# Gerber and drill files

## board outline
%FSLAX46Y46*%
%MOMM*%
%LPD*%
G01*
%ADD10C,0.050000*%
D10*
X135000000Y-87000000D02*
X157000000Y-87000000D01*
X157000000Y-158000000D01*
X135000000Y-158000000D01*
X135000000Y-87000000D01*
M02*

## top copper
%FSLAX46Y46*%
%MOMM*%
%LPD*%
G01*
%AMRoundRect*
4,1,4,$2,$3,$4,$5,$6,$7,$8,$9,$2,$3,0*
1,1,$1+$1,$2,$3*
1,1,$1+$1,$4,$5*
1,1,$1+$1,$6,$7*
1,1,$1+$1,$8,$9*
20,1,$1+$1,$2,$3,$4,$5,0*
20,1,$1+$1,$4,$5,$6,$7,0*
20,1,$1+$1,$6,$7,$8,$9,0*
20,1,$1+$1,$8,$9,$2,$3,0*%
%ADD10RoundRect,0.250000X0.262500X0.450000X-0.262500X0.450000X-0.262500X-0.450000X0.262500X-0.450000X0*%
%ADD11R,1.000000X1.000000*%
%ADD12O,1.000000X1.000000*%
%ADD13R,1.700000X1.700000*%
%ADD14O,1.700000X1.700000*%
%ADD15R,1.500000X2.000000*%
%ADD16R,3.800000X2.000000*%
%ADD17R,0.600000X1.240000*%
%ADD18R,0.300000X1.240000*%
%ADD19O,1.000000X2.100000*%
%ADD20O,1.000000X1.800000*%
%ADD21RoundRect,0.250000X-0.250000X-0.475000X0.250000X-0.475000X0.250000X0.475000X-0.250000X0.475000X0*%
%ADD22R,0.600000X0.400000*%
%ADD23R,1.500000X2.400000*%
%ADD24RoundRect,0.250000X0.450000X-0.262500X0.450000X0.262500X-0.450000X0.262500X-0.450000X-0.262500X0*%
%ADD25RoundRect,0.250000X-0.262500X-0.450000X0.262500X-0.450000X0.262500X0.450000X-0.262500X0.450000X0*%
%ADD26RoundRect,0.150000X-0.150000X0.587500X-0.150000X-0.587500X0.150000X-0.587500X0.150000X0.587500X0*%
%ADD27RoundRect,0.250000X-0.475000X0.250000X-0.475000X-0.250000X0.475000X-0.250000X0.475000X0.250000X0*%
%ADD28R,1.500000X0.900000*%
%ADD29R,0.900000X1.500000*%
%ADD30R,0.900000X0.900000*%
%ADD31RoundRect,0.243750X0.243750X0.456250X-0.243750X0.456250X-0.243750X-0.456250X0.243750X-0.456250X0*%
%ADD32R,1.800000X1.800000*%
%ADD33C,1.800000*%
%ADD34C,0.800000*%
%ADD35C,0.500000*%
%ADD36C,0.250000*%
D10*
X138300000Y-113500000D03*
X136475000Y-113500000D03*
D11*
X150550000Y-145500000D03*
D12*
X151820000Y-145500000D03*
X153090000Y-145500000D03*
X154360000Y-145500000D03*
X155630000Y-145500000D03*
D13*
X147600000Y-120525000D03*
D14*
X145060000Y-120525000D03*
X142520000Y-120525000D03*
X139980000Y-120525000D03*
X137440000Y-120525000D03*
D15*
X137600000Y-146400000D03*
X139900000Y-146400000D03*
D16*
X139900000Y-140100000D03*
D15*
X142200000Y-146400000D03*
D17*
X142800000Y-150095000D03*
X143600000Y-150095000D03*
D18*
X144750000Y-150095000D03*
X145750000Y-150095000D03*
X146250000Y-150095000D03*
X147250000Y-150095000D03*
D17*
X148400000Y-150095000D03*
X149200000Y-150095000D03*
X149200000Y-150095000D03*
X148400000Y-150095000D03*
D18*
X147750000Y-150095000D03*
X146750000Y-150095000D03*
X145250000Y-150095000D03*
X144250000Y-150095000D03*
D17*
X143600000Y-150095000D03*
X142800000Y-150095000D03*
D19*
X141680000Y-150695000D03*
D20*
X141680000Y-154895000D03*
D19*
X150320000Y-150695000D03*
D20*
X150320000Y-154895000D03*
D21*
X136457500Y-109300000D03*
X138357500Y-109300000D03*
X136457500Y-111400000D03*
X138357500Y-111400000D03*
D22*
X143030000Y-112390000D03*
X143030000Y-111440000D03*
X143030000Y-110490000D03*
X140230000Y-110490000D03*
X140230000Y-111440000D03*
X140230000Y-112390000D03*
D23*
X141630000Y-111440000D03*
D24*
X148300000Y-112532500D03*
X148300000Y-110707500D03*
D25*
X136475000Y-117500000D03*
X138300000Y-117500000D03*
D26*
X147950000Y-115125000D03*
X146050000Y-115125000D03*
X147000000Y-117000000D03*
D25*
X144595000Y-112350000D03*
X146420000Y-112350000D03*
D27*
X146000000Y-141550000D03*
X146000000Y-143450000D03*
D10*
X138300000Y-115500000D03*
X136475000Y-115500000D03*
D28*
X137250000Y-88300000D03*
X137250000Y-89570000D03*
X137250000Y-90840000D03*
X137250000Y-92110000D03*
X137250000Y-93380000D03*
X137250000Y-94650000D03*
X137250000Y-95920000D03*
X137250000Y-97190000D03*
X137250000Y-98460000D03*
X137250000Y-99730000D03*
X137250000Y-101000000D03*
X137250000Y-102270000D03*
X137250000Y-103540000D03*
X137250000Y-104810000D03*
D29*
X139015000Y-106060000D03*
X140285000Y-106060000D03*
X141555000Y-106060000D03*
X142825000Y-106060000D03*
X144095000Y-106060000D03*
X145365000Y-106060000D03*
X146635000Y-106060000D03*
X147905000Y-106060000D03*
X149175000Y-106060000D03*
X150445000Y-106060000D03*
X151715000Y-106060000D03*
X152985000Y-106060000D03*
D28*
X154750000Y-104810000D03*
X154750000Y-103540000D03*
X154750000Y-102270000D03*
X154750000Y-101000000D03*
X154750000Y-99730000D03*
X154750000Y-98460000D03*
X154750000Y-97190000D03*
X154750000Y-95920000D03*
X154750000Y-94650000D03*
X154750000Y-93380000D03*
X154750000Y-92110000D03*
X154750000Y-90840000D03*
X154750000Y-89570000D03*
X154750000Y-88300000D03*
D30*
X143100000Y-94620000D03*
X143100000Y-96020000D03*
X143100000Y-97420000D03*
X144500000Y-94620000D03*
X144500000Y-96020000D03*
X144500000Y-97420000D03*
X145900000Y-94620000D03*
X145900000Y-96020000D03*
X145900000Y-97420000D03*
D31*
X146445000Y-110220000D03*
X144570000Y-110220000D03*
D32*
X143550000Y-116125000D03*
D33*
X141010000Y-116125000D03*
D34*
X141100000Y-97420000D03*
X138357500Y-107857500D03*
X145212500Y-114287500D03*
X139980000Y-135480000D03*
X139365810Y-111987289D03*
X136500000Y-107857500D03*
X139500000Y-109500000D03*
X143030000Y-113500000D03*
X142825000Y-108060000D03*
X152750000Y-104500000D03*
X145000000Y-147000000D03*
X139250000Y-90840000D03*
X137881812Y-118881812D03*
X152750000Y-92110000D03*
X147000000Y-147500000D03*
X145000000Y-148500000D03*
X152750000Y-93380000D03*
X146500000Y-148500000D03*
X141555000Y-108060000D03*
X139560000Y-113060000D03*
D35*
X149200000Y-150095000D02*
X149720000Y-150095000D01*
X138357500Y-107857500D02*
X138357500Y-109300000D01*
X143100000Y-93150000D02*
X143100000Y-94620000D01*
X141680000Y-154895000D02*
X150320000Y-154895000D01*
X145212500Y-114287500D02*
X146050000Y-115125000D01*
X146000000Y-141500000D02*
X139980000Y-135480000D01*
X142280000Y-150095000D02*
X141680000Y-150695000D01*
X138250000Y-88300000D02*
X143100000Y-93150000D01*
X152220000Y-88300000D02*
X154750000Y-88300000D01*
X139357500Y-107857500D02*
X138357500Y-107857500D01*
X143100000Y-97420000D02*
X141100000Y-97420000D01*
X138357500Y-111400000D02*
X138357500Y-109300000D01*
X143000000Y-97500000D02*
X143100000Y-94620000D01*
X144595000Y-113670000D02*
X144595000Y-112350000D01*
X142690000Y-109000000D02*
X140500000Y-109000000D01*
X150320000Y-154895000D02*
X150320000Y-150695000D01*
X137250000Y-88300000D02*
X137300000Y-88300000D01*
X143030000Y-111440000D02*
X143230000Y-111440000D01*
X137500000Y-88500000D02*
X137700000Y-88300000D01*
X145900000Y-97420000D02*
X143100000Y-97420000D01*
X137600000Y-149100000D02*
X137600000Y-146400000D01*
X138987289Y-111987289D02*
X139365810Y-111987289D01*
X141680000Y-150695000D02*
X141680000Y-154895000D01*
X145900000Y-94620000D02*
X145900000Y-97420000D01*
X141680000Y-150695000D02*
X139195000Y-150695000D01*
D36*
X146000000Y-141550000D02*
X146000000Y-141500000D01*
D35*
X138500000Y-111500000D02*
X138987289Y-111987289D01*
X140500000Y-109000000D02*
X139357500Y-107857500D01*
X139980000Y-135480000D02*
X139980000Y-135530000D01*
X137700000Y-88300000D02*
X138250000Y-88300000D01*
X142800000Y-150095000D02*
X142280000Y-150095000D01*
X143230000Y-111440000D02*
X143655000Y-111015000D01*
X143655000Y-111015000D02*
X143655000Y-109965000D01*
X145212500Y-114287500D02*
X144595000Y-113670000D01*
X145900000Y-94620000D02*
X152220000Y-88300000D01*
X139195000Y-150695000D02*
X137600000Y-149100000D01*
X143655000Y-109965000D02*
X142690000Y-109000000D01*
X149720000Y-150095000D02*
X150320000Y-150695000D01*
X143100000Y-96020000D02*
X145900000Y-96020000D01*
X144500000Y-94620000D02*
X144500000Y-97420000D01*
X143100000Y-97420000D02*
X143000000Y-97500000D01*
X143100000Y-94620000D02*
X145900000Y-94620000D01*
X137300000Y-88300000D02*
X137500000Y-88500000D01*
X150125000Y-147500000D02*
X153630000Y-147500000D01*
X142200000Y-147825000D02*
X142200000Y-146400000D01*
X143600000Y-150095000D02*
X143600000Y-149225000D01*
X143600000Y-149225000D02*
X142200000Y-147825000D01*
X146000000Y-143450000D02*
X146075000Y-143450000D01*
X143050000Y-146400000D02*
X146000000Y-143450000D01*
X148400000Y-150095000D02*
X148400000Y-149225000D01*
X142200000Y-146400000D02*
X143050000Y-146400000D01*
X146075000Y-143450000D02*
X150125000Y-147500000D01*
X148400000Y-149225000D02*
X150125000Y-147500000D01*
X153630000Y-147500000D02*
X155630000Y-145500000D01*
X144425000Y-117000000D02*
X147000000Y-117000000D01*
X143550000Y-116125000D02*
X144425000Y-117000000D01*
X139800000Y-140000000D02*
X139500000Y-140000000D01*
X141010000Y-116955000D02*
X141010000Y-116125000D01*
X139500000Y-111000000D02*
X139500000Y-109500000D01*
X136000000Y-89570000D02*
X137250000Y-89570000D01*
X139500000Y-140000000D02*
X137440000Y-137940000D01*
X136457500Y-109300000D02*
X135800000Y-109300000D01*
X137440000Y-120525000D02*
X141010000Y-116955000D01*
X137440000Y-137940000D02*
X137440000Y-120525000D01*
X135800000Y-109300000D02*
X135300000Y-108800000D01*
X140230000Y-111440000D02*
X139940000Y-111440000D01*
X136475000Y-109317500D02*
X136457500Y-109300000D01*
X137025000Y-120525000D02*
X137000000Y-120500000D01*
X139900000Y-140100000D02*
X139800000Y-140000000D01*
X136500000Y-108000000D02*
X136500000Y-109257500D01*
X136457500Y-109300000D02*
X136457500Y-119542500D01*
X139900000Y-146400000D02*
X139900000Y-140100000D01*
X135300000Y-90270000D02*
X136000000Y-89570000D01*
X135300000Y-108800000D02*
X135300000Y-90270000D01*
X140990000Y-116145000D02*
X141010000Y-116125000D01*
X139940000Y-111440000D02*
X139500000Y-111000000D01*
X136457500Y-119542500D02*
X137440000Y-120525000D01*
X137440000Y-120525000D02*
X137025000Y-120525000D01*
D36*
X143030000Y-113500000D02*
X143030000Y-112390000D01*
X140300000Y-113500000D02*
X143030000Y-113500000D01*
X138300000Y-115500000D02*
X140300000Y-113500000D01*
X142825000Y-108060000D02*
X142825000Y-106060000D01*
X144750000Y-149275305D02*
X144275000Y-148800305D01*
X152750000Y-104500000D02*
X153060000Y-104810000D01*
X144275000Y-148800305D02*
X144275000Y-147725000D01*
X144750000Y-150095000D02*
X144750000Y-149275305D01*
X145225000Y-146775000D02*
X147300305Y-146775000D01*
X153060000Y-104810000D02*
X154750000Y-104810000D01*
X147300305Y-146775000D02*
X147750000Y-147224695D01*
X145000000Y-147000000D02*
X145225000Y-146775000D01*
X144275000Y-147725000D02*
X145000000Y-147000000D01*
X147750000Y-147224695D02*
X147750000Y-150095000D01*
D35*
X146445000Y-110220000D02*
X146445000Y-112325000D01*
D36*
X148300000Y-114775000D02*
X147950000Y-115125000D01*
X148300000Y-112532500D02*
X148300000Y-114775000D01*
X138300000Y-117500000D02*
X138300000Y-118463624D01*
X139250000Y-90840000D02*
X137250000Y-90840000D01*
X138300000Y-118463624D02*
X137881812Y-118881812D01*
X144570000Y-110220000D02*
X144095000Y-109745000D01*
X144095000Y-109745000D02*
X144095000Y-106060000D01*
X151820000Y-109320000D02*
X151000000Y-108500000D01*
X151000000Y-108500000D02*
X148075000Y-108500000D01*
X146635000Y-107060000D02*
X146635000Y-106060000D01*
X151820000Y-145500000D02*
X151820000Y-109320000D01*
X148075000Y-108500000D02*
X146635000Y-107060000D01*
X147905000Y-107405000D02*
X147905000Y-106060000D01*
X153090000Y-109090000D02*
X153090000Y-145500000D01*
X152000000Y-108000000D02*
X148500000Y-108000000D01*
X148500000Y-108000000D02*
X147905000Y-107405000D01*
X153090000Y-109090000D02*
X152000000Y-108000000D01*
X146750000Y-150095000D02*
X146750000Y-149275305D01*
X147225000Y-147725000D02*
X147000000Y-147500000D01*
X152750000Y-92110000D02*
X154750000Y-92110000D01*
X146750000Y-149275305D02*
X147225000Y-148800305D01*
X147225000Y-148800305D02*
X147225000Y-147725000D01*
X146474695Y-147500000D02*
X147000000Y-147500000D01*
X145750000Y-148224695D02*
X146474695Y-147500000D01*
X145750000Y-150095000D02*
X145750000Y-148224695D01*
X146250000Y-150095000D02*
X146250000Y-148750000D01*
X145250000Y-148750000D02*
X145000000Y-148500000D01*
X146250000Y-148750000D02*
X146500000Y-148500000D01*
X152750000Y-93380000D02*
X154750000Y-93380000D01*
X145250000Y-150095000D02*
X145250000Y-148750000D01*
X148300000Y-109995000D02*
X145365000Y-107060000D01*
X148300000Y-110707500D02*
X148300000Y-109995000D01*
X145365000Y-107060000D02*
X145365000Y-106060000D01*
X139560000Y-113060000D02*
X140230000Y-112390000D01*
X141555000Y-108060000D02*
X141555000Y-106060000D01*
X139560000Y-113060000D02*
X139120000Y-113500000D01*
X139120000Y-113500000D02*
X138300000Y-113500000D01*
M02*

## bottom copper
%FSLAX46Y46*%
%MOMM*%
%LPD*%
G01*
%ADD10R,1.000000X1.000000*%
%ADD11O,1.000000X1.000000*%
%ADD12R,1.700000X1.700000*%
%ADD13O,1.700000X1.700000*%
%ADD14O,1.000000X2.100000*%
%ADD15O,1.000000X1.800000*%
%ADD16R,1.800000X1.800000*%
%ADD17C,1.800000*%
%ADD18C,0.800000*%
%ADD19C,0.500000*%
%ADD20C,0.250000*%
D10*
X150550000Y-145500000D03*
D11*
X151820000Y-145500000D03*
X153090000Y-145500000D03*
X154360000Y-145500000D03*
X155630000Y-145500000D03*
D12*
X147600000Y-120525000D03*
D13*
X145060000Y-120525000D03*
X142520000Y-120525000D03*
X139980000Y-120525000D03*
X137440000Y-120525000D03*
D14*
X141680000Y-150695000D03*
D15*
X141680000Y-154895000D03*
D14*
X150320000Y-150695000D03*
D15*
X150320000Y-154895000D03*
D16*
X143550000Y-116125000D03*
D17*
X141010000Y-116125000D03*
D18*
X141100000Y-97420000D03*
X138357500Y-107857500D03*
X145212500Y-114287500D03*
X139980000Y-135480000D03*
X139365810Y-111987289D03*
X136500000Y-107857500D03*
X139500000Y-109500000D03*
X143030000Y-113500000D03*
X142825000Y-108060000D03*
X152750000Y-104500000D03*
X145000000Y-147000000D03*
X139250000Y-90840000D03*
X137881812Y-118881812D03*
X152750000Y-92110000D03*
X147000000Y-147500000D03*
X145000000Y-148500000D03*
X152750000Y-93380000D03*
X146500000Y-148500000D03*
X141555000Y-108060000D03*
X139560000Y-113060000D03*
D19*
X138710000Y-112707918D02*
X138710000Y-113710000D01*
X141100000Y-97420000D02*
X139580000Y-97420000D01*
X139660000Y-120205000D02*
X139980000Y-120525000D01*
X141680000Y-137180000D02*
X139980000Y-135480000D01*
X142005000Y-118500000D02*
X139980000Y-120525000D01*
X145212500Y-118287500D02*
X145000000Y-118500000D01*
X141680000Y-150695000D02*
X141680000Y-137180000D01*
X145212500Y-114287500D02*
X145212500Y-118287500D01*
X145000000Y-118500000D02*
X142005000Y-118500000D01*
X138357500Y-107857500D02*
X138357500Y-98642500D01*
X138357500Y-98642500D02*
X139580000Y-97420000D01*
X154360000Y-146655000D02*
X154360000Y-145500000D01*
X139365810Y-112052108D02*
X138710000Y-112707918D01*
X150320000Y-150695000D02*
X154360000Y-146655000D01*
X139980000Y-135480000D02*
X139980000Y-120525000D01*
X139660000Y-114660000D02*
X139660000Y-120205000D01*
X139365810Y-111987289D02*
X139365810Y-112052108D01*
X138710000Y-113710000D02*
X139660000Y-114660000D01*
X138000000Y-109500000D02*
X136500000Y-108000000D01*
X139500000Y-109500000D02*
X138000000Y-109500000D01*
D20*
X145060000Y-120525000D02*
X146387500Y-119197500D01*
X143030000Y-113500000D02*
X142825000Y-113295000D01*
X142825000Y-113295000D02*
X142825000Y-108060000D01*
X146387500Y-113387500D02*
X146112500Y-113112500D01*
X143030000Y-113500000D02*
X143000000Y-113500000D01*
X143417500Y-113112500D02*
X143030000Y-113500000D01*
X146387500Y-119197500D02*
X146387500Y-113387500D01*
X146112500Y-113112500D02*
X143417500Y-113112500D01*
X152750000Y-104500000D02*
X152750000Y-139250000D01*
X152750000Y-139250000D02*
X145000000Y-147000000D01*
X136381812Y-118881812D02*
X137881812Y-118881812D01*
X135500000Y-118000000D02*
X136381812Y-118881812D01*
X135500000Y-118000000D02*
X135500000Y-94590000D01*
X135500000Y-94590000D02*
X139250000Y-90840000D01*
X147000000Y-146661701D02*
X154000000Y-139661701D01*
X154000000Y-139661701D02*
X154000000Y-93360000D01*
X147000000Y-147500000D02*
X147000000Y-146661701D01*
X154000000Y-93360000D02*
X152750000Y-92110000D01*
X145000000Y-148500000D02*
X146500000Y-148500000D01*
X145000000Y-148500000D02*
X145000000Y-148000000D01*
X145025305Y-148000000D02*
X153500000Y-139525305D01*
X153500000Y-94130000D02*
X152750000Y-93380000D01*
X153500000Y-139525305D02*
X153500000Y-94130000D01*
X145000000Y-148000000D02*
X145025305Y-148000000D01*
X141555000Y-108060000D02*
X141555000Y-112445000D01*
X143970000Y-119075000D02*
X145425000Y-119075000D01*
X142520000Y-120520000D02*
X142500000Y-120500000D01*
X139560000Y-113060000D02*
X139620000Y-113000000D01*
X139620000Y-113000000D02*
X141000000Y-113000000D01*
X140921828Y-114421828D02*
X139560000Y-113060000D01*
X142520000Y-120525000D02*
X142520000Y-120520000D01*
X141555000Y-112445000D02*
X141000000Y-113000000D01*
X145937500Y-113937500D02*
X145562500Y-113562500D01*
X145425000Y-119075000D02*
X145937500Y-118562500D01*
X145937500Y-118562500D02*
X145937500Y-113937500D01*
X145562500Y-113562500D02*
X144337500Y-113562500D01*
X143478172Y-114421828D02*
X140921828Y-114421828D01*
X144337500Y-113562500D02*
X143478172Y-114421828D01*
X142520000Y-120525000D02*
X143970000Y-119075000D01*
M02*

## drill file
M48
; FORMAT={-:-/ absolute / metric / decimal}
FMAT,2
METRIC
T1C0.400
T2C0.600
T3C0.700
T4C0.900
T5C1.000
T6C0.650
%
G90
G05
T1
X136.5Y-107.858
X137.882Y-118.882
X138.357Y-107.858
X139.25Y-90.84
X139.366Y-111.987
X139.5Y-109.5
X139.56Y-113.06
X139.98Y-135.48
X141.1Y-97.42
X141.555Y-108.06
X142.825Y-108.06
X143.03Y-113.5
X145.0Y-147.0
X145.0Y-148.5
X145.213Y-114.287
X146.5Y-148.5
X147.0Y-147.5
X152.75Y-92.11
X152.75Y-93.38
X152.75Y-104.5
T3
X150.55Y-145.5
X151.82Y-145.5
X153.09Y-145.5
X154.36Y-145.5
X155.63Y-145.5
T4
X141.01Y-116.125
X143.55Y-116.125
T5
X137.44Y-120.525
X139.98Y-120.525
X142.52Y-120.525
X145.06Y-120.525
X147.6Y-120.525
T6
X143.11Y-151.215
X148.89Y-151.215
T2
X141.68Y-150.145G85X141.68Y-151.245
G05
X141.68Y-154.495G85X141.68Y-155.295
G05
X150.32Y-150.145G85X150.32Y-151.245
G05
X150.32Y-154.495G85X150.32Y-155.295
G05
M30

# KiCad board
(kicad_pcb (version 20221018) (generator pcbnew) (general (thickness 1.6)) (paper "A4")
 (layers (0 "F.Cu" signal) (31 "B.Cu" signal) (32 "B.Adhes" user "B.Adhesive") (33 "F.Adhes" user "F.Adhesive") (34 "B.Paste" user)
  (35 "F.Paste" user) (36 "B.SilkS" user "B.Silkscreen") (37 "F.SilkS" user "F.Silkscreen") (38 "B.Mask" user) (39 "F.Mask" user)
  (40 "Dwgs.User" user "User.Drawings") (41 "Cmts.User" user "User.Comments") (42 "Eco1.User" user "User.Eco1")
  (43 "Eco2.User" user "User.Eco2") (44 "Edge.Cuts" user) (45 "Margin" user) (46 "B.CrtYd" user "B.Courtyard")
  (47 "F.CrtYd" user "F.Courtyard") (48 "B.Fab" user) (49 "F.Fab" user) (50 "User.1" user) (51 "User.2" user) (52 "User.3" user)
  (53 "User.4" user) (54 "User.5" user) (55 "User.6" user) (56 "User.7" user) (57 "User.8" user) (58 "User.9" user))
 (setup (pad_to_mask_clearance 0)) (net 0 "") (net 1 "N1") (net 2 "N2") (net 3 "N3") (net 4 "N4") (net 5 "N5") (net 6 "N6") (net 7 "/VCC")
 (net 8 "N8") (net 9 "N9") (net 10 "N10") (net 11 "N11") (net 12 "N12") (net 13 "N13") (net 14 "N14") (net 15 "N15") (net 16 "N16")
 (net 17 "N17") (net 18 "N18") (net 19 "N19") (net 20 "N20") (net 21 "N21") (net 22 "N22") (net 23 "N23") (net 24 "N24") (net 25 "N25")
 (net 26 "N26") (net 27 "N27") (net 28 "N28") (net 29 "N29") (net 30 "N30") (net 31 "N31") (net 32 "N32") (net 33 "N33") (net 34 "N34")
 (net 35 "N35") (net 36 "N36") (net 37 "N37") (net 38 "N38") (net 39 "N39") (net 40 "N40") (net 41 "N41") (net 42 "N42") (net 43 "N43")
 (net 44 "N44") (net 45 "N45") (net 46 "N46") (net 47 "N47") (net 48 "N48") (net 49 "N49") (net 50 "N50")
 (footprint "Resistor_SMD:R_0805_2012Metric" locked (layer "F.Cu") (at 137.3875 113.5 180)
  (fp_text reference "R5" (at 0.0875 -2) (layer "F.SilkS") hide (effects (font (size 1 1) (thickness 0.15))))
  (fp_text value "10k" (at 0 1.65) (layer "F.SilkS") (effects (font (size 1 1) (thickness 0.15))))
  (pad "1" smd roundrect locked (at -0.9125 0 180) (size 1.025 1.4) (layers "F.Cu" "F.Paste" "F.Mask") (roundrect_rratio 0.243902439)
   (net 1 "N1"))
  (pad "2" smd roundrect locked (at 0.9125 0 180) (size 1.025 1.4) (layers "F.Cu" "F.Paste" "F.Mask") (roundrect_rratio 0.243902439)
   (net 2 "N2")))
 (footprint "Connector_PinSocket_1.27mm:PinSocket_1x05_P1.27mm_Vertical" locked (layer "F.Cu") (at 150.55 145.5 90)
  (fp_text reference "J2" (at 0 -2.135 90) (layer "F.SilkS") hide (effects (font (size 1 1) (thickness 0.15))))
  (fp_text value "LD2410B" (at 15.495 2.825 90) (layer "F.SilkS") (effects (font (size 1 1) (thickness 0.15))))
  (pad "1" thru_hole rect locked (at 0 0 90) (size 1 1) (drill 0.7) (layers "*.Cu" "*.Mask") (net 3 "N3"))
  (pad "2" thru_hole oval locked (at 0 1.27 90) (size 1 1) (drill 0.7) (layers "*.Cu" "*.Mask") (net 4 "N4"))
  (pad "3" thru_hole oval locked (at 0 2.54 90) (size 1 1) (drill 0.7) (layers "*.Cu" "*.Mask") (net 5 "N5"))
  (pad "4" thru_hole oval locked (at 0 3.81 90) (size 1 1) (drill 0.7) (layers "*.Cu" "*.Mask") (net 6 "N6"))
  (pad "5" thru_hole oval locked (at 0 5.08 90) (size 1 1) (drill 0.7) (layers "*.Cu" "*.Mask") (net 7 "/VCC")))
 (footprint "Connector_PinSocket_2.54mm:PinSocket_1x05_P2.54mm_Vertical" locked (layer "F.Cu") (at 147.6 120.525 -90)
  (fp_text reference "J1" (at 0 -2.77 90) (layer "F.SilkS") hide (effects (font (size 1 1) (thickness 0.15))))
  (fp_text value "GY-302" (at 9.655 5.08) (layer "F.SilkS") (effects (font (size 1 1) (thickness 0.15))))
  (pad "1" thru_hole rect locked (at 0 0 270) (size 1.7 1.7) (drill 1) (layers "*.Cu" "*.Mask") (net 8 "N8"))
  (pad "2" thru_hole oval locked (at 0 2.54 270) (size 1.7 1.7) (drill 1) (layers "*.Cu" "*.Mask") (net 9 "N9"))
  (pad "3" thru_hole oval locked (at 0 5.08 270) (size 1.7 1.7) (drill 1) (layers "*.Cu" "*.Mask") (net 1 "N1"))
  (pad "4" thru_hole oval locked (at 0 7.62 270) (size 1.7 1.7) (drill 1) (layers "*.Cu" "*.Mask") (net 6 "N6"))
  (pad "5" thru_hole oval locked (at 0 10.16 270) (size 1.7 1.7) (drill 1) (layers "*.Cu" "*.Mask") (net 2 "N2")))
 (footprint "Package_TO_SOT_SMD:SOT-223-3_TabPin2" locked (layer "F.Cu") (at 139.9 143.25 90)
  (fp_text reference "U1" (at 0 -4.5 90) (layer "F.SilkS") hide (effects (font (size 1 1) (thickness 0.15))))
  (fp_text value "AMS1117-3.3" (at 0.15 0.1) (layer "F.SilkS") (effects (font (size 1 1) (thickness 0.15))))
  (pad "1" smd rect locked (at -3.15 -2.3 90) (size 2 1.5) (layers "F.Cu" "F.Paste" "F.Mask") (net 6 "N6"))
  (pad "2" smd rect locked (at -3.15 0 90) (size 2 1.5) (layers "F.Cu" "F.Paste" "F.Mask") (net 2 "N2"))
  (pad "2" smd rect locked (at 3.15 0 90) (size 2 3.8) (layers "F.Cu" "F.Paste" "F.Mask") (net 2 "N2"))
  (pad "3" smd rect locked (at -3.15 2.3 90) (size 2 1.5) (layers "F.Cu" "F.Paste" "F.Mask") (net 7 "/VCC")))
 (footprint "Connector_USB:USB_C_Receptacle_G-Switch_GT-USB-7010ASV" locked (layer "F.Cu") (at 146 153.82)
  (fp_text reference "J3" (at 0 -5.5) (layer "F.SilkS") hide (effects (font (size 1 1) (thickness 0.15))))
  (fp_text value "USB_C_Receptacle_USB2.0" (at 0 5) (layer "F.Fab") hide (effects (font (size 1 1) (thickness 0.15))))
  (pad "" np_thru_hole circle locked (at -2.89 -2.605) (size 0.65 0.65) (drill 0.65) (layers "*.Cu" "*.Mask"))
  (pad "" np_thru_hole circle locked (at 2.89 -2.605) (size 0.65 0.65) (drill 0.65) (layers "*.Cu" "*.Mask"))
  (pad "A1" smd rect locked (at -3.2 -3.725) (size 0.6 1.24) (layers "F.Cu" "F.Paste" "F.Mask") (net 6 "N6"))
  (pad "A4" smd rect locked (at -2.4 -3.725) (size 0.6 1.24) (layers "F.Cu" "F.Paste" "F.Mask") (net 7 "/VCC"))
  (pad "A5" smd rect locked (at -1.25 -3.725) (size 0.3 1.24) (layers "F.Cu" "F.Paste" "F.Mask") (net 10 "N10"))
  (pad "A6" smd rect locked (at -0.25 -3.725) (size 0.3 1.24) (layers "F.Cu" "F.Paste" "F.Mask") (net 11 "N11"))
  (pad "A7" smd rect locked (at 0.25 -3.725) (size 0.3 1.24) (layers "F.Cu" "F.Paste" "F.Mask") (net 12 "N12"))
  (pad "A8" smd rect locked (at 1.25 -3.725) (size 0.3 1.24) (layers "F.Cu" "F.Paste" "F.Mask") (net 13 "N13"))
  (pad "A9" smd rect locked (at 2.4 -3.725) (size 0.6 1.24) (layers "F.Cu" "F.Paste" "F.Mask") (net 7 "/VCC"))
  (pad "A12" smd rect locked (at 3.2 -3.725) (size 0.6 1.24) (layers "F.Cu" "F.Paste" "F.Mask") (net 6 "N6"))
  (pad "B1" smd rect locked (at 3.2 -3.725) (size 0.6 1.24) (layers "F.Cu" "F.Paste" "F.Mask") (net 6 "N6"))
  (pad "B4" smd rect locked (at 2.4 -3.725) (size 0.6 1.24) (layers "F.Cu" "F.Paste" "F.Mask") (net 7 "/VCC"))
  (pad "B5" smd rect locked (at 1.75 -3.725) (size 0.3 1.24) (layers "F.Cu" "F.Paste" "F.Mask") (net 10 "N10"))
  (pad "B6" smd rect locked (at 0.75 -3.725) (size 0.3 1.24) (layers "F.Cu" "F.Paste" "F.Mask") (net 11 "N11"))
  (pad "B7" smd rect locked (at -0.75 -3.725) (size 0.3 1.24) (layers "F.Cu" "F.Paste" "F.Mask") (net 12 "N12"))
  (pad "B8" smd rect locked (at -1.75 -3.725) (size 0.3 1.24) (layers "F.Cu" "F.Paste" "F.Mask") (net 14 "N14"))
  (pad "B9" smd rect locked (at -2.4 -3.725) (size 0.6 1.24) (layers "F.Cu" "F.Paste" "F.Mask") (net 7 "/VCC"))
  (pad "B12" smd rect locked (at -3.2 -3.725) (size 0.6 1.24) (layers "F.Cu" "F.Paste" "F.Mask") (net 6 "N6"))
  (pad "S1" thru_hole oval locked (at -4.32 -3.125) (size 1 2.1) (drill oval 0.6 1.7) (layers "*.Cu" "*.Mask") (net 6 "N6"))
  (pad "S1" thru_hole oval locked (at -4.32 1.075) (size 1 1.8) (drill oval 0.6 1.4) (layers "*.Cu" "*.Mask") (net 6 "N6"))
  (pad "S1" thru_hole oval locked (at 4.32 -3.125) (size 1 2.1) (drill oval 0.6 1.7) (layers "*.Cu" "*.Mask") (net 6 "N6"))
  (pad "S1" thru_hole oval locked (at 4.32 1.075) (size 1 1.8) (drill oval 0.6 1.4) (layers "*.Cu" "*.Mask") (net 6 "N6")))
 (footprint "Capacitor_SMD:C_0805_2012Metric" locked (layer "F.Cu") (at 137.4075 109.3)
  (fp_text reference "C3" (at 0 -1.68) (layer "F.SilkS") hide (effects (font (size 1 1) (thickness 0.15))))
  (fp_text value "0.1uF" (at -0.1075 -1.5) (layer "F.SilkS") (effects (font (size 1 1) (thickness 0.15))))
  (pad "1" smd roundrect locked (at -0.95 0) (size 1 1.45) (layers "F.Cu" "F.Paste" "F.Mask") (roundrect_rratio 0.25) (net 2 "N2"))
  (pad "2" smd roundrect locked (at 0.95 0) (size 1 1.45) (layers "F.Cu" "F.Paste" "F.Mask") (roundrect_rratio 0.25) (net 6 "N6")))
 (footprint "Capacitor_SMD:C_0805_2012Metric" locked (layer "F.Cu") (at 137.4075 111.4)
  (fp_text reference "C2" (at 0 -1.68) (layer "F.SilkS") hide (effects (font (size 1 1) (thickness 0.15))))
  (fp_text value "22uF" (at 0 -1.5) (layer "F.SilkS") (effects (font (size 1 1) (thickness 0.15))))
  (pad "1" smd roundrect locked (at -0.95 0) (size 1 1.45) (layers "F.Cu" "F.Paste" "F.Mask") (roundrect_rratio 0.25) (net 2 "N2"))
  (pad "2" smd roundrect locked (at 0.95 0) (size 1 1.45) (layers "F.Cu" "F.Paste" "F.Mask") (roundrect_rratio 0.25) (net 6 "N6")))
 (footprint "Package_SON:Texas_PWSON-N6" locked (layer "F.Cu") (at 141.63 111.44 180)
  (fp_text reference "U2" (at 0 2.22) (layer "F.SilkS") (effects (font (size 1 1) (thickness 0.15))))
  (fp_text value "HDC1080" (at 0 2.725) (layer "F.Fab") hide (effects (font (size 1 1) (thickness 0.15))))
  (pad "1" smd rect locked (at -1.4 -0.95 180) (size 0.6 0.4) (layers "F.Cu" "F.Paste" "F.Mask") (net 9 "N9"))
  (pad "2" smd rect locked (at -1.4 0 180) (size 0.6 0.4) (layers "F.Cu" "F.Paste" "F.Mask") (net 6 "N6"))
  (pad "3" smd rect locked (at -1.4 0.95 180) (size 0.6 0.4) (layers "F.Cu" "F.Paste" "F.Mask") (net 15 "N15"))
  (pad "4" smd rect locked (at 1.4 0.95 180) (size 0.6 0.4) (layers "F.Cu" "F.Paste" "F.Mask") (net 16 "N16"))
  (pad "5" smd rect locked (at 1.4 0 180) (size 0.6 0.4) (layers "F.Cu" "F.Paste" "F.Mask") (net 2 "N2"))
  (pad "6" smd rect locked (at 1.4 -0.95 180) (size 0.6 0.4) (layers "F.Cu" "F.Paste" "F.Mask") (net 1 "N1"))
  (pad "7" smd rect locked (at 0 0 180) (size 1.5 2.4) (layers "F.Cu" "F.Paste" "F.Mask") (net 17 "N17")))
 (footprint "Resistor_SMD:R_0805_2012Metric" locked (layer "F.Cu") (at 148.3 111.62 90)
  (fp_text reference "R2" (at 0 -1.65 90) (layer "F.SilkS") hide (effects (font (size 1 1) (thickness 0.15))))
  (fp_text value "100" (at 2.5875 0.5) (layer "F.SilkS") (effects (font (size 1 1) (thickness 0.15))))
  (pad "1" smd roundrect locked (at -0.9125 0 90) (size 1.025 1.4) (layers "F.Cu" "F.Paste" "F.Mask") (roundrect_rratio 0.243902439)
   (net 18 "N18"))
  (pad "2" smd roundrect locked (at 0.9125 0 90) (size 1.025 1.4) (layers "F.Cu" "F.Paste" "F.Mask") (roundrect_rratio 0.243902439)
   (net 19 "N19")))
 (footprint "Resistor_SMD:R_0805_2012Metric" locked (layer "F.Cu") (at 137.3875 117.5)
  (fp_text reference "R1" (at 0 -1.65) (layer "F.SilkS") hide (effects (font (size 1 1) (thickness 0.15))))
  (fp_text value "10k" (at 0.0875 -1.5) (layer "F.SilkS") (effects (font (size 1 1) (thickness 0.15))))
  (pad "1" smd roundrect locked (at -0.9125 0) (size 1.025 1.4) (layers "F.Cu" "F.Paste" "F.Mask") (roundrect_rratio 0.243902439)
   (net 2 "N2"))
  (pad "2" smd roundrect locked (at 0.9125 0) (size 1.025 1.4) (layers "F.Cu" "F.Paste" "F.Mask") (roundrect_rratio 0.243902439)
   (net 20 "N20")))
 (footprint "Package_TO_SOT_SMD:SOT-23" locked (layer "F.Cu") (at 147 116.0625 -90)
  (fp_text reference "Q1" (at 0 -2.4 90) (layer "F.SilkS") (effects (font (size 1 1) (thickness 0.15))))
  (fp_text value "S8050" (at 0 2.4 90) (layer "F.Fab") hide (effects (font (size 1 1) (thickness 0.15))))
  (pad "1" smd roundrect locked (at -0.9375 -0.95 270) (size 1.475 0.6) (layers "F.Cu" "F.Paste" "F.Mask") (roundrect_rratio 0.25)
   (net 18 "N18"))
  (pad "2" smd roundrect locked (at -0.9375 0.95 270) (size 1.475 0.6) (layers "F.Cu" "F.Paste" "F.Mask") (roundrect_rratio 0.25)
   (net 6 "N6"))
  (pad "3" smd roundrect locked (at 0.9375 0 270) (size 1.475 0.6) (layers "F.Cu" "F.Paste" "F.Mask") (roundrect_rratio 0.25) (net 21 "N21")))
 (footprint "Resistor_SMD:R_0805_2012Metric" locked (layer "F.Cu") (at 145.5075 112.35)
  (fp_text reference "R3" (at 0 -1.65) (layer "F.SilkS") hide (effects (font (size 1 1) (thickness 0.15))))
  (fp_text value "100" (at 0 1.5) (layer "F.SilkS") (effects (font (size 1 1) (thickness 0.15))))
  (pad "1" smd roundrect locked (at -0.9125 0) (size 1.025 1.4) (layers "F.Cu" "F.Paste" "F.Mask") (roundrect_rratio 0.243902439)
   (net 6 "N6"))
  (pad "2" smd roundrect locked (at 0.9125 0) (size 1.025 1.4) (layers "F.Cu" "F.Paste" "F.Mask") (roundrect_rratio 0.243902439)
   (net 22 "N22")))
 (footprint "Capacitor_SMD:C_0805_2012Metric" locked (layer "F.Cu") (at 146 142.5 -90)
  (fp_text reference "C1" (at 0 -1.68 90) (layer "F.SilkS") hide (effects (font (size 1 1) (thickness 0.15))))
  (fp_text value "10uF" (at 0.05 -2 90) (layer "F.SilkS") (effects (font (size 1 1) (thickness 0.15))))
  (pad "1" smd roundrect locked (at -0.95 0 270) (size 1 1.45) (layers "F.Cu" "F.Paste" "F.Mask") (roundrect_rratio 0.25) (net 6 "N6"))
  (pad "2" smd roundrect locked (at 0.95 0 270) (size 1 1.45) (layers "F.Cu" "F.Paste" "F.Mask") (roundrect_rratio 0.25) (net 7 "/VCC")))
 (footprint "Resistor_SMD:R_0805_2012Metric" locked (layer "F.Cu") (at 137.3875 115.5 180)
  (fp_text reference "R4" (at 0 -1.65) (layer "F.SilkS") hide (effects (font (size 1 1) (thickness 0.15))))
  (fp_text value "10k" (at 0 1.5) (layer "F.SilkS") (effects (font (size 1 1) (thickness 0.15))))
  (pad "1" smd roundrect locked (at -0.9125 0 180) (size 1.025 1.4) (layers "F.Cu" "F.Paste" "F.Mask") (roundrect_rratio 0.243902439)
   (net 9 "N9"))
  (pad "2" smd roundrect locked (at 0.9125 0 180) (size 1.025 1.4) (layers "F.Cu" "F.Paste" "F.Mask") (roundrect_rratio 0.243902439)
   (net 2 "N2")))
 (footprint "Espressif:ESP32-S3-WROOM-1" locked (layer "F.Cu") (at 146 96.56)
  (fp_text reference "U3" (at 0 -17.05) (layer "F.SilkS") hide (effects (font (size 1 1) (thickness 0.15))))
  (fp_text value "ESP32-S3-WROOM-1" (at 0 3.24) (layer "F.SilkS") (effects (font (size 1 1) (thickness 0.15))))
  (pad "1" smd rect locked (at -8.75 -8.26) (size 1.5 0.9) (layers "F.Cu" "F.Paste" "F.Mask") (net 6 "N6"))
  (pad "2" smd rect locked (at -8.75 -6.99) (size 1.5 0.9) (layers "F.Cu" "F.Paste" "F.Mask") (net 2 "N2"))
  (pad "3" smd rect locked (at -8.75 -5.72) (size 1.5 0.9) (layers "F.Cu" "F.Paste" "F.Mask") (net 20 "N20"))
  (pad "4" smd rect locked (at -8.75 -4.45) (size 1.5 0.9) (layers "F.Cu" "F.Paste" "F.Mask") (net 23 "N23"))
  (pad "5" smd rect locked (at -8.75 -3.18) (size 1.5 0.9) (layers "F.Cu" "F.Paste" "F.Mask") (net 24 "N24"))
  (pad "6" smd rect locked (at -8.75 -1.91) (size 1.5 0.9) (layers "F.Cu" "F.Paste" "F.Mask") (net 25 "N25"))
  (pad "7" smd rect locked (at -8.75 -0.64) (size 1.5 0.9) (layers "F.Cu" "F.Paste" "F.Mask") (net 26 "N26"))
  (pad "8" smd rect locked (at -8.75 0.63) (size 1.5 0.9) (layers "F.Cu" "F.Paste" "F.Mask") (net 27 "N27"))
  (pad "9" smd rect locked (at -8.75 1.9) (size 1.5 0.9) (layers "F.Cu" "F.Paste" "F.Mask") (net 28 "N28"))
  (pad "10" smd rect locked (at -8.75 3.17) (size 1.5 0.9) (layers "F.Cu" "F.Paste" "F.Mask") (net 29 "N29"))
  (pad "11" smd rect locked (at -8.75 4.44) (size 1.5 0.9) (layers "F.Cu" "F.Paste" "F.Mask") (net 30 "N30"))
  (pad "12" smd rect locked (at -8.75 5.71) (size 1.5 0.9) (layers "F.Cu" "F.Paste" "F.Mask") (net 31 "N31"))
  (pad "13" smd rect locked (at -8.75 6.98) (size 1.5 0.9) (layers "F.Cu" "F.Paste" "F.Mask") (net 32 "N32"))
  (pad "14" smd rect locked (at -8.75 8.25) (size 1.5 0.9) (layers "F.Cu" "F.Paste" "F.Mask") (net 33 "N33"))
  (pad "15" smd rect locked (at -6.985 9.5 90) (size 1.5 0.9) (layers "F.Cu" "F.Paste" "F.Mask") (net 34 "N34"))
  (pad "16" smd rect locked (at -5.715 9.5 90) (size 1.5 0.9) (layers "F.Cu" "F.Paste" "F.Mask") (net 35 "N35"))
  (pad "17" smd rect locked (at -4.445 9.5 90) (size 1.5 0.9) (layers "F.Cu" "F.Paste" "F.Mask") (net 1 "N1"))
  (pad "18" smd rect locked (at -3.175 9.5 90) (size 1.5 0.9) (layers "F.Cu" "F.Paste" "F.Mask") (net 9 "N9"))
  (pad "19" smd rect locked (at -1.905 9.5 90) (size 1.5 0.9) (layers "F.Cu" "F.Paste" "F.Mask") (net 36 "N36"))
  (pad "20" smd rect locked (at -0.635 9.5 90) (size 1.5 0.9) (layers "F.Cu" "F.Paste" "F.Mask") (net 19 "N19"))
  (pad "21" smd rect locked (at 0.635 9.5 90) (size 1.5 0.9) (layers "F.Cu" "F.Paste" "F.Mask") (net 4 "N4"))
  (pad "22" smd rect locked (at 1.905 9.5 90) (size 1.5 0.9) (layers "F.Cu" "F.Paste" "F.Mask") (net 5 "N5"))
  (pad "23" smd rect locked (at 3.175 9.5 90) (size 1.5 0.9) (layers "F.Cu" "F.Paste" "F.Mask") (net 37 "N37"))
  (pad "24" smd rect locked (at 4.445 9.5 90) (size 1.5 0.9) (layers "F.Cu" "F.Paste" "F.Mask") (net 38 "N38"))
  (pad "25" smd rect locked (at 5.715 9.5 90) (size 1.5 0.9) (layers "F.Cu" "F.Paste" "F.Mask") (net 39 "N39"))
  (pad "26" smd rect locked (at 6.985 9.5 90) (size 1.5 0.9) (layers "F.Cu" "F.Paste" "F.Mask") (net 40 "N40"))
  (pad "27" smd rect locked (at 8.75 8.25 180) (size 1.5 0.9) (layers "F.Cu" "F.Paste" "F.Mask") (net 10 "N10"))
  (pad "28" smd rect locked (at 8.75 6.98 180) (size 1.5 0.9) (layers "F.Cu" "F.Paste" "F.Mask") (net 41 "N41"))
  (pad "29" smd rect locked (at 8.75 5.71 180) (size 1.5 0.9) (layers "F.Cu" "F.Paste" "F.Mask") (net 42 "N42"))
  (pad "30" smd rect locked (at 8.75 4.44 180) (size 1.5 0.9) (layers "F.Cu" "F.Paste" "F.Mask") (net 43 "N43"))
  (pad "31" smd rect locked (at 8.75 3.17 180) (size 1.5 0.9) (layers "F.Cu" "F.Paste" "F.Mask") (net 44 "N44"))
  (pad "32" smd rect locked (at 8.75 1.9 180) (size 1.5 0.9) (layers "F.Cu" "F.Paste" "F.Mask") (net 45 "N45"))
  (pad "33" smd rect locked (at 8.75 0.63 180) (size 1.5 0.9) (layers "F.Cu" "F.Paste" "F.Mask") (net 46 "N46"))
  (pad "34" smd rect locked (at 8.75 -0.64 180) (size 1.5 0.9) (layers "F.Cu" "F.Paste" "F.Mask") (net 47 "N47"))
  (pad "35" smd rect locked (at 8.75 -1.91 180) (size 1.5 0.9) (layers "F.Cu" "F.Paste" "F.Mask") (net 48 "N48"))
  (pad "36" smd rect locked (at 8.75 -3.18 180) (size 1.5 0.9) (layers "F.Cu" "F.Paste" "F.Mask") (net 12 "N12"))
  (pad "37" smd rect locked (at 8.75 -4.45 180) (size 1.5 0.9) (layers "F.Cu" "F.Paste" "F.Mask") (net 11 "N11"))
  (pad "38" smd rect locked (at 8.75 -5.72 180) (size 1.5 0.9) (layers "F.Cu" "F.Paste" "F.Mask") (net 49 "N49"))
  (pad "39" smd rect locked (at 8.75 -6.99 180) (size 1.5 0.9) (layers "F.Cu" "F.Paste" "F.Mask") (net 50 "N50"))
  (pad "40" smd rect locked (at 8.75 -8.26 180) (size 1.5 0.9) (layers "F.Cu" "F.Paste" "F.Mask") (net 6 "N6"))
  (pad "41" smd rect locked (at -2.9 -1.94 180) (size 0.9 0.9) (layers "F.Cu" "F.Paste" "F.Mask") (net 6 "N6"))
  (pad "41" smd rect locked (at -2.9 -0.54 180) (size 0.9 0.9) (layers "F.Cu" "F.Paste" "F.Mask") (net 6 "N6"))
  (pad "41" smd rect locked (at -2.9 0.86 180) (size 0.9 0.9) (layers "F.Cu" "F.Paste" "F.Mask") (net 6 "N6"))
  (pad "41" smd rect locked (at -1.5 -1.94 180) (size 0.9 0.9) (layers "F.Cu" "F.Paste" "F.Mask") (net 6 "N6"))
  (pad "41" smd rect locked (at -1.5 -0.54 180) (size 0.9 0.9) (layers "F.Cu" "F.Paste" "F.Mask") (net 6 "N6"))
  (pad "41" smd rect locked (at -1.5 0.86 180) (size 0.9 0.9) (layers "F.Cu" "F.Paste" "F.Mask") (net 6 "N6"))
  (pad "41" smd rect locked (at -0.1 -1.94 180) (size 0.9 0.9) (layers "F.Cu" "F.Paste" "F.Mask") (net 6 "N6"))
  (pad "41" smd rect locked (at -0.1 -0.54 180) (size 0.9 0.9) (layers "F.Cu" "F.Paste" "F.Mask") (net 6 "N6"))
  (pad "41" smd rect locked (at -0.1 0.86 180) (size 0.9 0.9) (layers "F.Cu" "F.Paste" "F.Mask") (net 6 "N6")))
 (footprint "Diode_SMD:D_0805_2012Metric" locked (layer "F.Cu") (at 145.5075 110.22 180)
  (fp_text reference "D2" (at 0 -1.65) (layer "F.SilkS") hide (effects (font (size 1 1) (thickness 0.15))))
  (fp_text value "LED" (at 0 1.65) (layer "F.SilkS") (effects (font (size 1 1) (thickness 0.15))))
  (pad "1" smd roundrect locked (at -0.9375 0 180) (size 0.975 1.4) (layers "F.Cu" "F.Paste" "F.Mask") (roundrect_rratio 0.25)
   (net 22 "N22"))
  (pad "2" smd roundrect locked (at 0.9375 0 180) (size 0.975 1.4) (layers "F.Cu" "F.Paste" "F.Mask") (roundrect_rratio 0.25) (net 36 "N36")))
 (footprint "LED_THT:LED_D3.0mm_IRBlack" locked (layer "F.Cu") (at 143.55 116.125 180)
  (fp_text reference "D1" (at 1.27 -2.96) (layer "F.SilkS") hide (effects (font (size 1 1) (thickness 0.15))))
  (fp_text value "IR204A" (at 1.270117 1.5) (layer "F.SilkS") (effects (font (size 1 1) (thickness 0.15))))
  (pad "1" thru_hole rect locked (at 0 0 180) (size 1.8 1.8) (drill 0.9) (layers "*.Cu" "*.Mask") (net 21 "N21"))
  (pad "2" thru_hole circle locked (at 2.54 0 180) (size 1.8 1.8) (drill 0.9) (layers "*.Cu" "*.Mask") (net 2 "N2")))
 (gr_rect locked (start 135 87) (end 157 158) (stroke (width 0.05) (type default)) (fill none) (layer "Edge.Cuts"))
 (segment (start 149.2 150.095) (end 149.72 150.095) (width 0.5) (layer "F.Cu") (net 6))
 (segment (start 138.3575 107.8575) (end 138.3575 109.3) (width 0.5) (layer "F.Cu") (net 6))
 (segment (start 143.1 93.15) (end 143.1 94.62) (width 0.5) (layer "F.Cu") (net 6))
 (segment (start 141.68 154.895) (end 150.32 154.895) (width 0.5) (layer "F.Cu") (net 6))
 (segment (start 145.2125 114.2875) (end 146.05 115.125) (width 0.5) (layer "F.Cu") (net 6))
 (segment (start 146 141.5) (end 139.98 135.48) (width 0.5) (layer "F.Cu") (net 6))
 (segment (start 142.28 150.095) (end 141.68 150.695) (width 0.5) (layer "F.Cu") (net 6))
 (segment (start 138.25 88.3) (end 143.1 93.15) (width 0.5) (layer "F.Cu") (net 6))
 (segment (start 152.22 88.3) (end 154.75 88.3) (width 0.5) (layer "F.Cu") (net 6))
 (segment (start 139.3575 107.8575) (end 138.3575 107.8575) (width 0.5) (layer "F.Cu") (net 6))
 (segment (start 143.1 97.42) (end 141.1 97.42) (width 0.5) (layer "F.Cu") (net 6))
 (segment (start 138.3575 111.4) (end 138.3575 109.3) (width 0.5) (layer "F.Cu") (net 6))
 (segment (start 143 97.5) (end 143.1 94.62) (width 0.5) (layer "F.Cu") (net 6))
 (segment (start 144.595 113.67) (end 144.595 112.35) (width 0.5) (layer "F.Cu") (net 6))
 (segment (start 142.69 109) (end 140.5 109) (width 0.5) (layer "F.Cu") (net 6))
 (segment (start 150.32 154.895) (end 150.32 150.695) (width 0.5) (layer "F.Cu") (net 6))
 (segment (start 137.25 88.3) (end 137.3 88.3) (width 0.5) (layer "F.Cu") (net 6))
 (segment (start 143.03 111.44) (end 143.23 111.44) (width 0.5) (layer "F.Cu") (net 6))
 (segment (start 137.5 88.5) (end 137.7 88.3) (width 0.5) (layer "F.Cu") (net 6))
 (segment (start 145.9 97.42) (end 143.1 97.42) (width 0.5) (layer "F.Cu") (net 6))
 (segment (start 137.6 149.1) (end 137.6 146.4) (width 0.5) (layer "F.Cu") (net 6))
 (segment (start 138.987289 111.987289) (end 139.36581 111.987289) (width 0.5) (layer "F.Cu") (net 6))
 (segment (start 141.68 150.695) (end 141.68 154.895) (width 0.5) (layer "F.Cu") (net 6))
 (segment (start 145.9 94.62) (end 145.9 97.42) (width 0.5) (layer "F.Cu") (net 6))
 (segment (start 141.68 150.695) (end 139.195 150.695) (width 0.5) (layer "F.Cu") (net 6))
 (segment (start 146 141.55) (end 146 141.5) (width 0.25) (layer "F.Cu") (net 6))
 (segment (start 138.5 111.5) (end 138.987289 111.987289) (width 0.5) (layer "F.Cu") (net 6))
 (segment (start 140.5 109) (end 139.3575 107.8575) (width 0.5) (layer "F.Cu") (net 6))
 (segment (start 139.98 135.48) (end 139.98 135.53) (width 0.5) (layer "F.Cu") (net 6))
 (segment (start 137.7 88.3) (end 138.25 88.3) (width 0.5) (layer "F.Cu") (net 6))
 (segment (start 142.8 150.095) (end 142.28 150.095) (width 0.5) (layer "F.Cu") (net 6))
 (segment (start 143.23 111.44) (end 143.655 111.015) (width 0.5) (layer "F.Cu") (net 6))
 (segment (start 143.655 111.015) (end 143.655 109.965) (width 0.5) (layer "F.Cu") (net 6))
 (segment (start 145.2125 114.2875) (end 144.595 113.67) (width 0.5) (layer "F.Cu") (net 6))
 (segment (start 145.9 94.62) (end 152.22 88.3) (width 0.5) (layer "F.Cu") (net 6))
 (segment (start 139.195 150.695) (end 137.6 149.1) (width 0.5) (layer "F.Cu") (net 6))
 (segment (start 143.655 109.965) (end 142.69 109) (width 0.5) (layer "F.Cu") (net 6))
 (segment (start 149.72 150.095) (end 150.32 150.695) (width 0.5) (layer "F.Cu") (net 6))
 (segment (start 143.1 96.02) (end 145.9 96.02) (width 0.5) (layer "F.Cu") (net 6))
 (segment (start 144.5 94.62) (end 144.5 97.42) (width 0.5) (layer "F.Cu") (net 6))
 (segment (start 143.1 97.42) (end 143 97.5) (width 0.5) (layer "F.Cu") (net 6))
 (segment (start 143.1 94.62) (end 145.9 94.62) (width 0.5) (layer "F.Cu") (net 6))
 (segment (start 137.3 88.3) (end 137.5 88.5) (width 0.5) (layer "F.Cu") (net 6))
 (via (at 141.1 97.42) (size 0.8) (drill 0.4) (layers "F.Cu" "B.Cu") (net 6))
 (via (at 138.3575 107.8575) (size 0.8) (drill 0.4) (layers "F.Cu" "B.Cu") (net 6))
 (via (at 145.2125 114.2875) (size 0.8) (drill 0.4) (layers "F.Cu" "B.Cu") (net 6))
 (via (at 139.98 135.48) (size 0.8) (drill 0.4) (layers "F.Cu" "B.Cu") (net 6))
 (via (at 139.36581 111.987289) (size 0.8) (drill 0.4) (layers "F.Cu" "B.Cu") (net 6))
 (segment (start 138.71 112.707918) (end 138.71 113.71) (width 0.5) (layer "B.Cu") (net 6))
 (segment (start 141.1 97.42) (end 139.58 97.42) (width 0.5) (layer "B.Cu") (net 6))
 (segment (start 139.66 120.205) (end 139.98 120.525) (width 0.5) (layer "B.Cu") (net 6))
 (segment (start 141.68 137.18) (end 139.98 135.48) (width 0.5) (layer "B.Cu") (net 6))
 (segment (start 142.005 118.5) (end 139.98 120.525) (width 0.5) (layer "B.Cu") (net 6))
 (segment (start 145.2125 118.2875) (end 145 118.5) (width 0.5) (layer "B.Cu") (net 6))
 (segment (start 141.68 150.695) (end 141.68 137.18) (width 0.5) (layer "B.Cu") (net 6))
 (segment (start 145.2125 114.2875) (end 145.2125 118.2875) (width 0.5) (layer "B.Cu") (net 6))
 (segment (start 145 118.5) (end 142.005 118.5) (width 0.5) (layer "B.Cu") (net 6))
 (segment (start 138.3575 107.8575) (end 138.3575 98.6425) (width 0.5) (layer "B.Cu") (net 6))
 (segment (start 138.3575 98.6425) (end 139.58 97.42) (width 0.5) (layer "B.Cu") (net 6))
 (segment (start 154.36 146.655) (end 154.36 145.5) (width 0.5) (layer "B.Cu") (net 6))
 (segment (start 139.36581 112.052108) (end 138.71 112.707918) (width 0.5) (layer "B.Cu") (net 6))
 (segment (start 150.32 150.695) (end 154.36 146.655) (width 0.5) (layer "B.Cu") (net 6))
 (segment (start 139.98 135.48) (end 139.98 120.525) (width 0.5) (layer "B.Cu") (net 6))
 (segment (start 139.66 114.66) (end 139.66 120.205) (width 0.5) (layer "B.Cu") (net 6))
 (segment (start 139.36581 111.987289) (end 139.36581 112.052108) (width 0.5) (layer "B.Cu") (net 6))
 (segment (start 138.71 113.71) (end 139.66 114.66) (width 0.5) (layer "B.Cu") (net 6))
 (segment (start 150.125 147.5) (end 153.63 147.5) (width 0.5) (layer "F.Cu") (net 7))
 (segment (start 142.2 147.825) (end 142.2 146.4) (width 0.5) (layer "F.Cu") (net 7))
 (segment (start 143.6 150.095) (end 143.6 149.225) (width 0.5) (layer "F.Cu") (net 7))
 (segment (start 143.6 149.225) (end 142.2 147.825) (width 0.5) (layer "F.Cu") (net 7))
 (segment (start 146 143.45) (end 146.075 143.45) (width 0.5) (layer "F.Cu") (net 7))
 (segment (start 143.05 146.4) (end 146 143.45) (width 0.5) (layer "F.Cu") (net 7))
 (segment (start 148.4 150.095) (end 148.4 149.225) (width 0.5) (layer "F.Cu") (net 7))
 (segment (start 142.2 146.4) (end 143.05 146.4) (width 0.5) (layer "F.Cu") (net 7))
 (segment (start 146.075 143.45) (end 150.125 147.5) (width 0.5) (layer "F.Cu") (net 7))
 (segment (start 148.4 149.225) (end 150.125 147.5) (width 0.5) (layer "F.Cu") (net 7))
 (segment (start 153.63 147.5) (end 155.63 145.5) (width 0.5) (layer "F.Cu") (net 7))
 (segment (start 144.425 117) (end 147 117) (width 0.5) (layer "F.Cu") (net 21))
 (segment (start 143.55 116.125) (end 144.425 117) (width 0.5) (layer "F.Cu") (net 21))
 (segment (start 139.8 140) (end 139.5 140) (width 0.5) (layer "F.Cu") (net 2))
 (segment (start 141.01 116.955) (end 141.01 116.125) (width 0.5) (layer "F.Cu") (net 2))
 (segment (start 139.5 111) (end 139.5 109.5) (width 0.5) (layer "F.Cu") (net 2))
 (segment (start 136 89.57) (end 137.25 89.57) (width 0.5) (layer "F.Cu") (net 2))
 (segment (start 139.5 140) (end 137.44 137.94) (width 0.5) (layer "F.Cu") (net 2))
 (segment (start 136.4575 109.3) (end 135.8 109.3) (width 0.5) (layer "F.Cu") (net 2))
 (segment (start 137.44 120.525) (end 141.01 116.955) (width 0.5) (layer "F.Cu") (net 2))
 (segment (start 137.44 137.94) (end 137.44 120.525) (width 0.5) (layer "F.Cu") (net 2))
 (segment (start 135.8 109.3) (end 135.3 108.8) (width 0.5) (layer "F.Cu") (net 2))
 (segment (start 140.23 111.44) (end 139.94 111.44) (width 0.5) (layer "F.Cu") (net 2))
 (segment (start 136.475 109.3175) (end 136.4575 109.3) (width 0.5) (layer "F.Cu") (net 2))
 (segment (start 137.025 120.525) (end 137 120.5) (width 0.5) (layer "F.Cu") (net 2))
 (segment (start 139.9 140.1) (end 139.8 140) (width 0.5) (layer "F.Cu") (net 2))
 (segment (start 136.5 108) (end 136.5 109.2575) (width 0.5) (layer "F.Cu") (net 2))
 (segment (start 136.4575 109.3) (end 136.4575 119.5425) (width 0.5) (layer "F.Cu") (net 2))
 (segment locked (start 139.9 146.4) (end 139.9 140.1) (width 0.5) (layer "F.Cu") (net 2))
 (segment (start 135.3 90.27) (end 136 89.57) (width 0.5) (layer "F.Cu") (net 2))
 (segment (start 135.3 108.8) (end 135.3 90.27) (width 0.5) (layer "F.Cu") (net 2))
 (segment (start 140.99 116.145) (end 141.01 116.125) (width 0.5) (layer "F.Cu") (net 2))
 (segment (start 139.94 111.44) (end 139.5 111) (width 0.5) (layer "F.Cu") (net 2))
 (segment (start 136.4575 119.5425) (end 137.44 120.525) (width 0.5) (layer "F.Cu") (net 2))
 (segment (start 137.44 120.525) (end 137.025 120.525) (width 0.5) (layer "F.Cu") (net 2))
 (via (at 136.5 107.8575) (size 0.8) (drill 0.4) (layers "F.Cu" "B.Cu") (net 2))
 (via (at 139.5 109.5) (size 0.8) (drill 0.4) (layers "F.Cu" "B.Cu") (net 2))
 (segment (start 138 109.5) (end 136.5 108) (width 0.5) (layer "B.Cu") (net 2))
 (segment (start 139.5 109.5) (end 138 109.5) (width 0.5) (layer "B.Cu") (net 2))
 (segment (start 143.03 113.5) (end 143.03 112.39) (width 0.25) (layer "F.Cu") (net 9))
 (segment (start 140.3 113.5) (end 143.03 113.5) (width 0.25) (layer "F.Cu") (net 9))
 (segment (start 138.3 115.5) (end 140.3 113.5) (width 0.25) (layer "F.Cu") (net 9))
 (segment (start 142.825 108.06) (end 142.825 106.06) (width 0.25) (layer "F.Cu") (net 9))
 (via (at 143.03 113.5) (size 0.8) (drill 0.4) (layers "F.Cu" "B.Cu") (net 9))
 (via (at 142.825 108.06) (size 0.8) (drill 0.4) (layers "F.Cu" "B.Cu") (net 9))
 (segment (start 145.06 120.525) (end 146.3875 119.1975) (width 0.25) (layer "B.Cu") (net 9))
 (segment (start 143.03 113.5) (end 142.825 113.295) (width 0.25) (layer "B.Cu") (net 9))
 (segment (start 142.825 113.295) (end 142.825 108.06) (width 0.25) (layer "B.Cu") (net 9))
 (segment (start 146.3875 113.3875) (end 146.1125 113.1125) (width 0.25) (layer "B.Cu") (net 9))
 (segment (start 143.03 113.5) (end 143 113.5) (width 0.25) (layer "B.Cu") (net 9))
 (segment (start 143.4175 113.1125) (end 143.03 113.5) (width 0.25) (layer "B.Cu") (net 9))
 (segment (start 146.3875 119.1975) (end 146.3875 113.3875) (width 0.25) (layer "B.Cu") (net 9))
 (segment (start 146.1125 113.1125) (end 143.4175 113.1125) (width 0.25) (layer "B.Cu") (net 9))
 (segment (start 144.75 149.275305) (end 144.275 148.800305) (width 0.25) (layer "F.Cu") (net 10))
 (segment (start 152.75 104.5) (end 153.06 104.81) (width 0.25) (layer "F.Cu") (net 10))
 (segment (start 144.275 148.800305) (end 144.275 147.725) (width 0.25) (layer "F.Cu") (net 10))
 (segment (start 144.75 150.095) (end 144.75 149.275305) (width 0.25) (layer "F.Cu") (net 10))
 (segment (start 145.225 146.775) (end 147.300305 146.775) (width 0.25) (layer "F.Cu") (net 10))
 (segment (start 153.06 104.81) (end 154.75 104.81) (width 0.25) (layer "F.Cu") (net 10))
 (segment (start 147.300305 146.775) (end 147.75 147.224695) (width 0.25) (layer "F.Cu") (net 10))
 (segment (start 145 147) (end 145.225 146.775) (width 0.25) (layer "F.Cu") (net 10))
 (segment (start 144.275 147.725) (end 145 147) (width 0.25) (layer "F.Cu") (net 10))
 (segment (start 147.75 147.224695) (end 147.75 150.095) (width 0.25) (layer "F.Cu") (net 10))
 (via (at 152.75 104.5) (size 0.8) (drill 0.4) (layers "F.Cu" "B.Cu") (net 10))
 (via (at 145 147) (size 0.8) (drill 0.4) (layers "F.Cu" "B.Cu") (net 10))
 (segment (start 152.75 104.5) (end 152.75 139.25) (width 0.25) (layer "B.Cu") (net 10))
 (segment (start 152.75 139.25) (end 145 147) (width 0.25) (layer "B.Cu") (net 10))
 (segment (start 146.445 110.22) (end 146.445 112.325) (width 0.5) (layer "F.Cu") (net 22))
 (segment (start 148.3 114.775) (end 147.95 115.125) (width 0.25) (layer "F.Cu") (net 18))
 (segment (start 148.3 112.5325) (end 148.3 114.775) (width 0.25) (layer "F.Cu") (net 18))
 (segment (start 138.3 117.5) (end 138.3 118.463624) (width 0.25) (layer "F.Cu") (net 20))
 (segment (start 139.25 90.84) (end 137.25 90.84) (width 0.25) (layer "F.Cu") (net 20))
 (segment (start 138.3 118.463624) (end 137.881812 118.881812) (width 0.25) (layer "F.Cu") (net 20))
 (via (at 139.25 90.84) (size 0.8) (drill 0.4) (layers "F.Cu" "B.Cu") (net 20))
 (via (at 137.881812 118.881812) (size 0.8) (drill 0.4) (layers "F.Cu" "B.Cu") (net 20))
 (segment (start 136.381812 118.881812) (end 137.881812 118.881812) (width 0.25) (layer "B.Cu") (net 20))
 (segment (start 135.5 118) (end 136.381812 118.881812) (width 0.25) (layer "B.Cu") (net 20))
 (segment (start 135.5 118) (end 135.5 94.59) (width 0.25) (layer "B.Cu") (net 20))
 (segment (start 135.5 94.59) (end 139.25 90.84) (width 0.25) (layer "B.Cu") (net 20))
 (segment (start 144.57 110.22) (end 144.095 109.745) (width 0.25) (layer "F.Cu") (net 36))
 (segment (start 144.095 109.745) (end 144.095 106.06) (width 0.25) (layer "F.Cu") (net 36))
 (segment (start 151.82 109.32) (end 151 108.5) (width 0.25) (layer "F.Cu") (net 4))
 (segment (start 151 108.5) (end 148.075 108.5) (width 0.25) (layer "F.Cu") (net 4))
 (segment (start 146.635 107.06) (end 146.635 106.06) (width 0.25) (layer "F.Cu") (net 4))
 (segment (start 151.82 145.5) (end 151.82 109.32) (width 0.25) (layer "F.Cu") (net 4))
 (segment (start 148.075 108.5) (end 146.635 107.06) (width 0.25) (layer "F.Cu") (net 4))
 (segment (start 147.905 107.405) (end 147.905 106.06) (width 0.25) (layer "F.Cu") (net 5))
 (segment (start 153.09 109.09) (end 153.09 145.5) (width 0.25) (layer "F.Cu") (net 5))
 (segment (start 152 108) (end 148.5 108) (width 0.25) (layer "F.Cu") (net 5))
 (segment (start 148.5 108) (end 147.905 107.405) (width 0.25) (layer "F.Cu") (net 5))
 (segment (start 153.09 109.09) (end 152 108) (width 0.25) (layer "F.Cu") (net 5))
 (segment (start 146.75 150.095) (end 146.75 149.275305) (width 0.25) (layer "F.Cu") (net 11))
 (segment (start 147.225 147.725) (end 147 147.5) (width 0.25) (layer "F.Cu") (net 11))
 (segment (start 152.75 92.11) (end 154.75 92.11) (width 0.25) (layer "F.Cu") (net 11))
 (segment (start 146.75 149.275305) (end 147.225 148.800305) (width 0.25) (layer "F.Cu") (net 11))
 (segment (start 147.225 148.800305) (end 147.225 147.725) (width 0.25) (layer "F.Cu") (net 11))
 (segment (start 146.474695 147.5) (end 147 147.5) (width 0.25) (layer "F.Cu") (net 11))
 (segment (start 145.75 148.224695) (end 146.474695 147.5) (width 0.25) (layer "F.Cu") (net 11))
 (segment (start 145.75 150.095) (end 145.75 148.224695) (width 0.25) (layer "F.Cu") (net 11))
 (via (at 152.75 92.11) (size 0.8) (drill 0.4) (layers "F.Cu" "B.Cu") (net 11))
 (via (at 147 147.5) (size 0.8) (drill 0.4) (layers "F.Cu" "B.Cu") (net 11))
 (segment (start 147 146.661701) (end 154 139.661701) (width 0.25) (layer "B.Cu") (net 11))
 (segment (start 154 139.661701) (end 154 93.36) (width 0.25) (layer "B.Cu") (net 11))
 (segment (start 147 147.5) (end 147 146.661701) (width 0.25) (layer "B.Cu") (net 11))
 (segment (start 154 93.36) (end 152.75 92.11) (width 0.25) (layer "B.Cu") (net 11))
 (segment (start 146.25 150.095) (end 146.25 148.75) (width 0.25) (layer "F.Cu") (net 12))
 (segment (start 145.25 148.75) (end 145 148.5) (width 0.25) (layer "F.Cu") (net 12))
 (segment (start 146.25 148.75) (end 146.5 148.5) (width 0.25) (layer "F.Cu") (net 12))
 (segment (start 152.75 93.38) (end 154.75 93.38) (width 0.25) (layer "F.Cu") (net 12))
 (segment (start 145.25 150.095) (end 145.25 148.75) (width 0.25) (layer "F.Cu") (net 12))
 (via (at 145 148.5) (size 0.8) (drill 0.4) (layers "F.Cu" "B.Cu") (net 12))
 (via (at 152.75 93.38) (size 0.8) (drill 0.4) (layers "F.Cu" "B.Cu") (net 12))
 (via (at 146.5 148.5) (size 0.8) (drill 0.4) (layers "F.Cu" "B.Cu") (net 12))
 (segment (start 145 148.5) (end 146.5 148.5) (width 0.25) (layer "B.Cu") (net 12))
 (segment (start 145 148.5) (end 145 148) (width 0.25) (layer "B.Cu") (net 12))
 (segment (start 145.025305 148) (end 153.5 139.525305) (width 0.25) (layer "B.Cu") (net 12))
 (segment (start 153.5 94.13) (end 152.75 93.38) (width 0.25) (layer "B.Cu") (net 12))
 (segment (start 153.5 139.525305) (end 153.5 94.13) (width 0.25) (layer "B.Cu") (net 12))
 (segment (start 145 148) (end 145.025305 148) (width 0.25) (layer "B.Cu") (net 12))
 (segment (start 148.3 109.995) (end 145.365 107.06) (width 0.25) (layer "F.Cu") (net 19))
 (segment (start 148.3 110.7075) (end 148.3 109.995) (width 0.25) (layer "F.Cu") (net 19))
 (segment (start 145.365 107.06) (end 145.365 106.06) (width 0.25) (layer "F.Cu") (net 19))
 (segment (start 139.56 113.06) (end 140.23 112.39) (width 0.25) (layer "F.Cu") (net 1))
 (segment (start 141.555 108.06) (end 141.555 106.06) (width 0.25) (layer "F.Cu") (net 1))
 (segment (start 139.56 113.06) (end 139.12 113.5) (width 0.25) (layer "F.Cu") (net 1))
 (segment (start 139.12 113.5) (end 138.3 113.5) (width 0.25) (layer "F.Cu") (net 1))
 (via (at 141.555 108.06) (size 0.8) (drill 0.4) (layers "F.Cu" "B.Cu") (free) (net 1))
 (via (at 139.56 113.06) (size 0.8) (drill 0.4) (layers "F.Cu" "B.Cu") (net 1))
 (segment (start 141.555 108.06) (end 141.555 112.445) (width 0.25) (layer "B.Cu") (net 1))
 (segment (start 143.97 119.075) (end 145.425 119.075) (width 0.25) (layer "B.Cu") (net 1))
 (segment (start 142.52 120.52) (end 142.5 120.5) (width 0.25) (layer "B.Cu") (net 1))
 (segment (start 139.56 113.06) (end 139.62 113) (width 0.25) (layer "B.Cu") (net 1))
 (segment (start 139.62 113) (end 141 113) (width 0.25) (layer "B.Cu") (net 1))
 (segment (start 140.921828 114.421828) (end 139.56 113.06) (width 0.25) (layer "B.Cu") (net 1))
 (segment (start 142.52 120.525) (end 142.52 120.52) (width 0.25) (layer "B.Cu") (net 1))
 (segment (start 141.555 112.445) (end 141 113) (width 0.25) (layer "B.Cu") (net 1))
 (segment (start 145.9375 113.9375) (end 145.5625 113.5625) (width 0.25) (layer "B.Cu") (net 1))
 (segment (start 145.425 119.075) (end 145.9375 118.5625) (width 0.25) (layer "B.Cu") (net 1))
 (segment (start 145.9375 118.5625) (end 145.9375 113.9375) (width 0.25) (layer "B.Cu") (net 1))
 (segment (start 145.5625 113.5625) (end 144.3375 113.5625) (width 0.25) (layer "B.Cu") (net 1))
 (segment (start 143.478172 114.421828) (end 140.921828 114.421828) (width 0.25) (layer "B.Cu") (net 1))
 (segment (start 144.3375 113.5625) (end 143.478172 114.421828) (width 0.25) (layer "B.Cu") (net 1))
 (segment (start 142.52 120.525) (end 143.97 119.075) (width 0.25) (layer "B.Cu") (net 1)))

